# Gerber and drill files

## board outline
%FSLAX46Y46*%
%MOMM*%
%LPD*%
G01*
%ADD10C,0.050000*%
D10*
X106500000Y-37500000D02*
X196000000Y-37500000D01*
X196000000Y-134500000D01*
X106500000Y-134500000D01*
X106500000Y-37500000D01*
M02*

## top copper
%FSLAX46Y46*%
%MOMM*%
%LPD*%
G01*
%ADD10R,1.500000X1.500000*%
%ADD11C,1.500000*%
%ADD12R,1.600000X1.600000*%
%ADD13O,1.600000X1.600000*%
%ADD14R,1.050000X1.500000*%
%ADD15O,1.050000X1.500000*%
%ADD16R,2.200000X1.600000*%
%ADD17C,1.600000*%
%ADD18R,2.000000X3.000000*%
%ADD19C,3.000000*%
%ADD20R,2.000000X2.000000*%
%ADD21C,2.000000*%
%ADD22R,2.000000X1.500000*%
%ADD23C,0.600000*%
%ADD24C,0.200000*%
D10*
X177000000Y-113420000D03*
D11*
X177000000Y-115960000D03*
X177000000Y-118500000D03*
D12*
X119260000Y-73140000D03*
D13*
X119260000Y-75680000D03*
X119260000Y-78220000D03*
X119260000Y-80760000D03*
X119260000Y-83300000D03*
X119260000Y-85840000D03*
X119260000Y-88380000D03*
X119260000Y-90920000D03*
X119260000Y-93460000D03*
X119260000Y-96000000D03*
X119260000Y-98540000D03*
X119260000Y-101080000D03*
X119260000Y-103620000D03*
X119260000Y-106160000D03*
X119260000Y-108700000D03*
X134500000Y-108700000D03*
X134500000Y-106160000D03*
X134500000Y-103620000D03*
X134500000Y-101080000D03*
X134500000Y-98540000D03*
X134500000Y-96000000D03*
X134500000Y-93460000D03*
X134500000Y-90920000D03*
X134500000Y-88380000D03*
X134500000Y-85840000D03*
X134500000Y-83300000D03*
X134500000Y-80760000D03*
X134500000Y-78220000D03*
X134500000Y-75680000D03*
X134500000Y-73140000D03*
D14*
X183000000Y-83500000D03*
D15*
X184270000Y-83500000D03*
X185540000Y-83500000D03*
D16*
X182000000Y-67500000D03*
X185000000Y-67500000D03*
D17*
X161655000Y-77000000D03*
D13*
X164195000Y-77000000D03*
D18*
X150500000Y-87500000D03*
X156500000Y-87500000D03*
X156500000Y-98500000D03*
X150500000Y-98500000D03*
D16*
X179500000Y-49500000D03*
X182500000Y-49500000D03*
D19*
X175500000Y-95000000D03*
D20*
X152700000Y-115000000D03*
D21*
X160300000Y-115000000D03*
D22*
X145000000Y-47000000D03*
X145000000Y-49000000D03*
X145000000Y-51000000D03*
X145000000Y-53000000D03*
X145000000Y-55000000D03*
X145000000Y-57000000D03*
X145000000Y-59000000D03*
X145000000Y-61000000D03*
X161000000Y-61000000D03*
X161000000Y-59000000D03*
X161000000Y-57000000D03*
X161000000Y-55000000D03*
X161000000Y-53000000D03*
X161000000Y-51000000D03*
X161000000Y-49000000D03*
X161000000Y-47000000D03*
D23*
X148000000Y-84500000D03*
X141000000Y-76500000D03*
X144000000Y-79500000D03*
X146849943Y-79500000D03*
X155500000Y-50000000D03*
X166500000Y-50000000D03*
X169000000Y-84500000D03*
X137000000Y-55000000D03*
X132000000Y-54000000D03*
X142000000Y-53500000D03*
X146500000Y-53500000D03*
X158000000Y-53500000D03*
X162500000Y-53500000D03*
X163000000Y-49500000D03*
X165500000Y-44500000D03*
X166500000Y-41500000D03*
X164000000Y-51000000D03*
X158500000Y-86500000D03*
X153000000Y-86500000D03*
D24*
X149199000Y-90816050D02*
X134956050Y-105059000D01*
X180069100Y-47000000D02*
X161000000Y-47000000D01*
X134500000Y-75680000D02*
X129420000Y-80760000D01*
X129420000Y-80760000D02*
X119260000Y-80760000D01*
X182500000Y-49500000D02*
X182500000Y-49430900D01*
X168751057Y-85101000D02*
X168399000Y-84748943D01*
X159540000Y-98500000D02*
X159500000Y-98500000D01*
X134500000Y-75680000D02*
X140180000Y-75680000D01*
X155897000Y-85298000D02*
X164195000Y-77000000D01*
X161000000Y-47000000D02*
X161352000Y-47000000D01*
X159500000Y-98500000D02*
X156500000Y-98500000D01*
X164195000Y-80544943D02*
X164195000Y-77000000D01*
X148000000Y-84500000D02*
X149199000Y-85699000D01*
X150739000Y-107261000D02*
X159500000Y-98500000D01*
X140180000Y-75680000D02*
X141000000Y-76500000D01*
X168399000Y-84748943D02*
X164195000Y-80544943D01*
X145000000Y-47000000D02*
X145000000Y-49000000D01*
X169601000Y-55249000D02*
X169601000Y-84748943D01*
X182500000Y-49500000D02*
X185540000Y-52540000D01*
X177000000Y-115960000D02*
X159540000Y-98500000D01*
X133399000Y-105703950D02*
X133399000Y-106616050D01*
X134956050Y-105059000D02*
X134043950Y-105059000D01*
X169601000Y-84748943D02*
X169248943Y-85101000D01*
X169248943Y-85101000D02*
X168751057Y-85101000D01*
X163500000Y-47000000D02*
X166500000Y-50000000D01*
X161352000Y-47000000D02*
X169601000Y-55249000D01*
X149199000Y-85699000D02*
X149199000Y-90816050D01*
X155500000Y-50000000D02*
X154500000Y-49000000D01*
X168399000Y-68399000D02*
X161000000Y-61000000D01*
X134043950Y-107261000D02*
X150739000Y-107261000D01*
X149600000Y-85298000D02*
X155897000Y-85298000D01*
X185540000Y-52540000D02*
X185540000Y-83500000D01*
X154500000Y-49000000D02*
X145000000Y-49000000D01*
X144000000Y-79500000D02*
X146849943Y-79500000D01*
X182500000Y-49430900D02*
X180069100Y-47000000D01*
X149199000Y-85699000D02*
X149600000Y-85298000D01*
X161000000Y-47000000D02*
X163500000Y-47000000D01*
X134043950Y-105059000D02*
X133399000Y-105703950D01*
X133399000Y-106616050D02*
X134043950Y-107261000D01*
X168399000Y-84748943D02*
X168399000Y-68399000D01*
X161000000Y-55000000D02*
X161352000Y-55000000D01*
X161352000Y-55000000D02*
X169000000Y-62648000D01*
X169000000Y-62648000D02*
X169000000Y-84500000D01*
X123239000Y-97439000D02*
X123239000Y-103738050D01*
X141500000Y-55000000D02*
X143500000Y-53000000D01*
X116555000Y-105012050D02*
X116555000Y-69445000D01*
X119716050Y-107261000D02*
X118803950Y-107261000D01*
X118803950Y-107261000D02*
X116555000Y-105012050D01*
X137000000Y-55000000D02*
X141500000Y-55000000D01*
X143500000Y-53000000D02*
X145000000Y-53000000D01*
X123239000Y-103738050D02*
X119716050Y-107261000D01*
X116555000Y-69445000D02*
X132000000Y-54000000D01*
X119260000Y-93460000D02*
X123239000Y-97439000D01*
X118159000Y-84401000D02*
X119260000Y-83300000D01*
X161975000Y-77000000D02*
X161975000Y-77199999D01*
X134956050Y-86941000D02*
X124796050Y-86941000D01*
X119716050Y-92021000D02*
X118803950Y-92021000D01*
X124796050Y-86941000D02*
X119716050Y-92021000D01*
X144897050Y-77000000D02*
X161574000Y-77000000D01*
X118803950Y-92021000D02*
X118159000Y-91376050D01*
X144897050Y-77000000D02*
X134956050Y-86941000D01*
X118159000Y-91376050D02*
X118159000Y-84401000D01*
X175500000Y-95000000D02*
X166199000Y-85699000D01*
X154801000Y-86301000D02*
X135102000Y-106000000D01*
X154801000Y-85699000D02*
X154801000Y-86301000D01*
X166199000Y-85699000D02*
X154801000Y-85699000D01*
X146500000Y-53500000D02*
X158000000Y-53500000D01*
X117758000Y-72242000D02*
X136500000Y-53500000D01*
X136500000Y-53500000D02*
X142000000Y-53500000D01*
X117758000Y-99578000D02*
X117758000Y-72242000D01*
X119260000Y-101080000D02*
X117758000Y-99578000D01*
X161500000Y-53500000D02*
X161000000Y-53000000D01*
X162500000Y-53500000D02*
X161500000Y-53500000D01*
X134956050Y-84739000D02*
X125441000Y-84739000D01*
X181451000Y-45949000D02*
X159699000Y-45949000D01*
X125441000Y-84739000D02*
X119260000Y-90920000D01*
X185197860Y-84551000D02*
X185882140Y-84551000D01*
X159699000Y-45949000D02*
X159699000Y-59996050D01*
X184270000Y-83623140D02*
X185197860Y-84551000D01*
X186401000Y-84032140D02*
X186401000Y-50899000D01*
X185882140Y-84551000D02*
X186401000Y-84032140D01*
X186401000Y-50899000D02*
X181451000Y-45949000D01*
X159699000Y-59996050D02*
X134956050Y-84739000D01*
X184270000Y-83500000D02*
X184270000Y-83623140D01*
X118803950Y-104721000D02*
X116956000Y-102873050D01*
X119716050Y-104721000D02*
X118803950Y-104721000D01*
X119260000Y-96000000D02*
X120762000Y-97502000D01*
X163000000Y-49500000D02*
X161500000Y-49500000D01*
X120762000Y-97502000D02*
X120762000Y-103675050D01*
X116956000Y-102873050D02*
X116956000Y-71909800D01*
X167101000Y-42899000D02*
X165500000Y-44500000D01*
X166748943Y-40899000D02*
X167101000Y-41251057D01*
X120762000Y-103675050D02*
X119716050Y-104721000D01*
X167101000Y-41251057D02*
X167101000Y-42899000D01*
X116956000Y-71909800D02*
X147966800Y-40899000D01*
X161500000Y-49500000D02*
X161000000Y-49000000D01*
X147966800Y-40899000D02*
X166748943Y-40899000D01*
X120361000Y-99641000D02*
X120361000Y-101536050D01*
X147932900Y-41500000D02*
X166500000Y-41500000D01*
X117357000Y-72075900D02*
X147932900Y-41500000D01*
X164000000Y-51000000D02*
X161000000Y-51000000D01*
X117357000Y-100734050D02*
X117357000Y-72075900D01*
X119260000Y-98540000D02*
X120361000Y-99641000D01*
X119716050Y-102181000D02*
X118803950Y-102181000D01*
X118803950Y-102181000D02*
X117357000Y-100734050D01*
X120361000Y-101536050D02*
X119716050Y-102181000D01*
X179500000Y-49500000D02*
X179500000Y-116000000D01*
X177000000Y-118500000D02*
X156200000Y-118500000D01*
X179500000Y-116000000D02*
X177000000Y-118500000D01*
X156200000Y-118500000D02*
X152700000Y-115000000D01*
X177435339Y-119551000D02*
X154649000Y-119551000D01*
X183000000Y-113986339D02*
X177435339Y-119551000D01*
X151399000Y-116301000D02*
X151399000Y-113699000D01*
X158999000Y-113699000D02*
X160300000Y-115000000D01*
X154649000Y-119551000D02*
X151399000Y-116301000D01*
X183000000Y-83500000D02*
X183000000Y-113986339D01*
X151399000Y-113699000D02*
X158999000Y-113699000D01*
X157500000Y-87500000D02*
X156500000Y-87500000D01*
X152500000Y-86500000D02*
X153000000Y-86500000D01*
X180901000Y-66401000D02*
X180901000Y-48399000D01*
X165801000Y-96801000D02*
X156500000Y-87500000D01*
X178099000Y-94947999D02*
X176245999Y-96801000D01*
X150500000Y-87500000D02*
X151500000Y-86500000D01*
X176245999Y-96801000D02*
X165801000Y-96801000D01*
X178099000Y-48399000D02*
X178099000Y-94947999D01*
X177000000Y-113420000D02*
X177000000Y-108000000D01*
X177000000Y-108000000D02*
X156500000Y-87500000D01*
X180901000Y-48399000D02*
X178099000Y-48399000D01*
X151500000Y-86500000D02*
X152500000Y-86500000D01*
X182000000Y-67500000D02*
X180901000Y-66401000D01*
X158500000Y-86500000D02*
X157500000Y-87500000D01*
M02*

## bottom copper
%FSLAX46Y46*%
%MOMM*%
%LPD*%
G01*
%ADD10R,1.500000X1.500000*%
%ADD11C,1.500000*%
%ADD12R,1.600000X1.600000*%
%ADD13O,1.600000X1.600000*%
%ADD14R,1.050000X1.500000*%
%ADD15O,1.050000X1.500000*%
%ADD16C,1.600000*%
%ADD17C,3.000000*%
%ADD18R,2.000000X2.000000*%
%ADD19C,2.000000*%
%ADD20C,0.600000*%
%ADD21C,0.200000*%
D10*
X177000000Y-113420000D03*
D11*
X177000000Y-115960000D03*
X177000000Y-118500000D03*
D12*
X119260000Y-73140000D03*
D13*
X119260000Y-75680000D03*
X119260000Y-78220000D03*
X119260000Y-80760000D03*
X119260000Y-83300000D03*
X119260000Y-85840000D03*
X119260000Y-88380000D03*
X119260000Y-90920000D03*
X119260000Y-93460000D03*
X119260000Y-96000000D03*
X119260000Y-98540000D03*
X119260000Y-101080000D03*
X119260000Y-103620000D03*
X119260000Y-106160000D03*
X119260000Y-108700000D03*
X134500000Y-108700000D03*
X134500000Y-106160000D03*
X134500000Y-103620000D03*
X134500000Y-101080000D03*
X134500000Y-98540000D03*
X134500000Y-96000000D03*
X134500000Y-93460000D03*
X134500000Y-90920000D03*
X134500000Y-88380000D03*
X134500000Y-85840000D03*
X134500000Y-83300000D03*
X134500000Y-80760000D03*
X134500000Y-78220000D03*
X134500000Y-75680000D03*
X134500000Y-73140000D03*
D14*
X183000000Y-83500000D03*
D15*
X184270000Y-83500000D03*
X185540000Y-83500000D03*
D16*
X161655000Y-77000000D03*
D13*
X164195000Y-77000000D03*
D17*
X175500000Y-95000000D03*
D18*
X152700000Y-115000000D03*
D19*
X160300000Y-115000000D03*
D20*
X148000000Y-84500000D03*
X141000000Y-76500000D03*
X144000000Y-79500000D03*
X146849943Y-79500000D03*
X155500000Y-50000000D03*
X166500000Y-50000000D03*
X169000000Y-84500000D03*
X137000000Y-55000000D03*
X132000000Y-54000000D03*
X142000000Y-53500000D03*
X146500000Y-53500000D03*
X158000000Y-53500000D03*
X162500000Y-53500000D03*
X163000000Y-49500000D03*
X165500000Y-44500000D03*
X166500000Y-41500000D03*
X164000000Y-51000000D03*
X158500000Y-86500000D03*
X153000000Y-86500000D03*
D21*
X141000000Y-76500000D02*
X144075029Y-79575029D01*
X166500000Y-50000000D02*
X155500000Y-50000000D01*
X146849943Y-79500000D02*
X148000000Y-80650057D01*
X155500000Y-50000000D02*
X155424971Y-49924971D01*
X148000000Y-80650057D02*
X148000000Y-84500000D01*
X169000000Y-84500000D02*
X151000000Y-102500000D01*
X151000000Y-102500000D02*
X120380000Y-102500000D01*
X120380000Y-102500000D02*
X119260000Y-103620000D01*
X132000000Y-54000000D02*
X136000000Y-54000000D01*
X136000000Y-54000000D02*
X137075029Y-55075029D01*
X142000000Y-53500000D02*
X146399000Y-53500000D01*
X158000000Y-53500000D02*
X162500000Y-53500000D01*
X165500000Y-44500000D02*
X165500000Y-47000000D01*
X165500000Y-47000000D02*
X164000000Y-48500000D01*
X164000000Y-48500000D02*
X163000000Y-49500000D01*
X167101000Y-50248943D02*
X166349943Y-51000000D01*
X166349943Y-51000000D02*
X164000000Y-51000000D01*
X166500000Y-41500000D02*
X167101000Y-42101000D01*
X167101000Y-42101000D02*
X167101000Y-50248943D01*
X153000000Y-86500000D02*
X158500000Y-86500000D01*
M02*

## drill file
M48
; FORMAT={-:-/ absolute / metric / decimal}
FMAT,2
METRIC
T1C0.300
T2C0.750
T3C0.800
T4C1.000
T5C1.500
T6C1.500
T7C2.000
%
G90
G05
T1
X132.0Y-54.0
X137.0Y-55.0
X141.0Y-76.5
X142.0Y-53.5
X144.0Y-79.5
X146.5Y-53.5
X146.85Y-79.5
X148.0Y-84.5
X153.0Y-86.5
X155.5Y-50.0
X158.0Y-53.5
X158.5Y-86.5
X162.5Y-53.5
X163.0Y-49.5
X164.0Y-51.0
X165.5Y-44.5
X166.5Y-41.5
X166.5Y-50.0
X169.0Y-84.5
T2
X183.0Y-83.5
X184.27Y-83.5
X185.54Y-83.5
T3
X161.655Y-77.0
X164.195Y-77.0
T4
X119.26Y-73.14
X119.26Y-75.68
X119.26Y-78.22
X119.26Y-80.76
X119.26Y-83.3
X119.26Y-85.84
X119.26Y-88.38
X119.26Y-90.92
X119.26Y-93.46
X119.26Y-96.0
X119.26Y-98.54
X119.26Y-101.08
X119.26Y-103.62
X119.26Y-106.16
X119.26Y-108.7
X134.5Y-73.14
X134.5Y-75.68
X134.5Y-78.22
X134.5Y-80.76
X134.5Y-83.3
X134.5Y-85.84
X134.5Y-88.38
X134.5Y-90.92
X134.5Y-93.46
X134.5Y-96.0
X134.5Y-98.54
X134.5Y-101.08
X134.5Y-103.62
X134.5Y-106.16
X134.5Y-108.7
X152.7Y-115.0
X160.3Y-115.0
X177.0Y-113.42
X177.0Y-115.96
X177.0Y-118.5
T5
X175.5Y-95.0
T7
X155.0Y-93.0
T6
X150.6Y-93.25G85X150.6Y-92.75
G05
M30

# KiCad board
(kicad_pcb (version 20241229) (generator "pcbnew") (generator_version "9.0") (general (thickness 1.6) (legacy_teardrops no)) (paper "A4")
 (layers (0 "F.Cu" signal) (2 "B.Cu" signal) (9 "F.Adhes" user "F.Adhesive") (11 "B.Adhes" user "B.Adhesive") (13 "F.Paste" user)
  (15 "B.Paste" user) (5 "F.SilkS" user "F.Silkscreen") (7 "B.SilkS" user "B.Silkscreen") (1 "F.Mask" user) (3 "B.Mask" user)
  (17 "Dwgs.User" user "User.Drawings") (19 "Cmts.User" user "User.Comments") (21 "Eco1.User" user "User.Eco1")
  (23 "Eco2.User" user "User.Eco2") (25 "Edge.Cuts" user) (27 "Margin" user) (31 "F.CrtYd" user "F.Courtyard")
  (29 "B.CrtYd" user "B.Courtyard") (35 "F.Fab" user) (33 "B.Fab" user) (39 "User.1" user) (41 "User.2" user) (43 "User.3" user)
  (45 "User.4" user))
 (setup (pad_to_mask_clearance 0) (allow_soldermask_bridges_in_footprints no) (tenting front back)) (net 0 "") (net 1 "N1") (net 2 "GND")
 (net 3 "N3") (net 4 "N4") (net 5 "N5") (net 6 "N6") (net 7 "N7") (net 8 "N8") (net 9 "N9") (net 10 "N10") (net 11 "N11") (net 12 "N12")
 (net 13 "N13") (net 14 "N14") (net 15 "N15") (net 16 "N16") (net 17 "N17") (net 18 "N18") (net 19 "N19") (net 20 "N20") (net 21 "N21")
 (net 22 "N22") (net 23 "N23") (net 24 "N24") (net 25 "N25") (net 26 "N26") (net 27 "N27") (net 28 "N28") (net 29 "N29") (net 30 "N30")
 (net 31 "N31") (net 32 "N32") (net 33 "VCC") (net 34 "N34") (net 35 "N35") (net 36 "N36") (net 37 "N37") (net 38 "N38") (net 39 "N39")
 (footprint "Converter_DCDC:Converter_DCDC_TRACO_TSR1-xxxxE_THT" (layer "F.Cu") (at 177 113.42)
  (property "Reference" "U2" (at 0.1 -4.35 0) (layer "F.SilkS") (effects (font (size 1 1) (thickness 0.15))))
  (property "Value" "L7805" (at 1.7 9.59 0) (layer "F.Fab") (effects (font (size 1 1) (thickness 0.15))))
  (pad "1" thru_hole rect (at 0 0) (size 1.5 1.5) (drill 1) (layers "*.Cu" "*.Mask") (remove_unused_layers no) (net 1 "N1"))
  (pad "2" thru_hole circle (at 0 2.54) (size 1.5 1.5) (drill 1) (layers "*.Cu" "*.Mask") (remove_unused_layers no) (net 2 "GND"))
  (pad "3" thru_hole circle (at 0 5.08) (size 1.5 1.5) (drill 1) (layers "*.Cu" "*.Mask") (remove_unused_layers no) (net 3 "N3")))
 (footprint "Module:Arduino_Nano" (layer "F.Cu") (at 119.26 73.14)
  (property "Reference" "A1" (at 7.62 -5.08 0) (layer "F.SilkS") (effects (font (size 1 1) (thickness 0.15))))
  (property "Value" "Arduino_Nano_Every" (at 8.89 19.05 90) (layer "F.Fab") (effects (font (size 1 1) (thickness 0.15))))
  (pad "1" thru_hole rect (at 0 0) (size 1.6 1.6) (drill 1) (layers "*.Cu" "*.Mask") (remove_unused_layers no) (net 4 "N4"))
  (pad "2" thru_hole oval (at 0 2.54) (size 1.6 1.6) (drill 1) (layers "*.Cu" "*.Mask") (remove_unused_layers no) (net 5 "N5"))
  (pad "3" thru_hole oval (at 0 5.08) (size 1.6 1.6) (drill 1) (layers "*.Cu" "*.Mask") (remove_unused_layers no) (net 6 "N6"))
  (pad "4" thru_hole oval (at 0 7.62) (size 1.6 1.6) (drill 1) (layers "*.Cu" "*.Mask") (remove_unused_layers no) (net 2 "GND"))
  (pad "5" thru_hole oval (at 0 10.16) (size 1.6 1.6) (drill 1) (layers "*.Cu" "*.Mask") (remove_unused_layers no) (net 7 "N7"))
  (pad "6" thru_hole oval (at 0 12.7) (size 1.6 1.6) (drill 1) (layers "*.Cu" "*.Mask") (remove_unused_layers no) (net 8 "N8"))
  (pad "7" thru_hole oval (at 0 15.24) (size 1.6 1.6) (drill 1) (layers "*.Cu" "*.Mask") (remove_unused_layers no) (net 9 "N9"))
  (pad "8" thru_hole oval (at 0 17.78) (size 1.6 1.6) (drill 1) (layers "*.Cu" "*.Mask") (remove_unused_layers no) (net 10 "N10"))
  (pad "9" thru_hole oval (at 0 20.32) (size 1.6 1.6) (drill 1) (layers "*.Cu" "*.Mask") (remove_unused_layers no) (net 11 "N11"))
  (pad "10" thru_hole oval (at 0 22.86) (size 1.6 1.6) (drill 1) (layers "*.Cu" "*.Mask") (remove_unused_layers no) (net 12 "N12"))
  (pad "11" thru_hole oval (at 0 25.4) (size 1.6 1.6) (drill 1) (layers "*.Cu" "*.Mask") (remove_unused_layers no) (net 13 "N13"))
  (pad "12" thru_hole oval (at 0 27.94) (size 1.6 1.6) (drill 1) (layers "*.Cu" "*.Mask") (remove_unused_layers no) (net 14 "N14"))
  (pad "13" thru_hole oval (at 0 30.48) (size 1.6 1.6) (drill 1) (layers "*.Cu" "*.Mask") (remove_unused_layers no) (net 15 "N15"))
  (pad "14" thru_hole oval (at 0 33.02) (size 1.6 1.6) (drill 1) (layers "*.Cu" "*.Mask") (remove_unused_layers no) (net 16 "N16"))
  (pad "15" thru_hole oval (at 0 35.56) (size 1.6 1.6) (drill 1) (layers "*.Cu" "*.Mask") (remove_unused_layers no) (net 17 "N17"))
  (pad "16" thru_hole oval (at 15.24 35.56) (size 1.6 1.6) (drill 1) (layers "*.Cu" "*.Mask") (remove_unused_layers no) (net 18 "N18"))
  (pad "17" thru_hole oval (at 15.24 33.02) (size 1.6 1.6) (drill 1) (layers "*.Cu" "*.Mask") (remove_unused_layers no) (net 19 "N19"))
  (pad "18" thru_hole oval (at 15.24 30.48) (size 1.6 1.6) (drill 1) (layers "*.Cu" "*.Mask") (remove_unused_layers no) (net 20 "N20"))
  (pad "19" thru_hole oval (at 15.24 27.94) (size 1.6 1.6) (drill 1) (layers "*.Cu" "*.Mask") (remove_unused_layers no) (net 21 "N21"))
  (pad "20" thru_hole oval (at 15.24 25.4) (size 1.6 1.6) (drill 1) (layers "*.Cu" "*.Mask") (remove_unused_layers no) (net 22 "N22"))
  (pad "21" thru_hole oval (at 15.24 22.86) (size 1.6 1.6) (drill 1) (layers "*.Cu" "*.Mask") (remove_unused_layers no) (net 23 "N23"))
  (pad "22" thru_hole oval (at 15.24 20.32) (size 1.6 1.6) (drill 1) (layers "*.Cu" "*.Mask") (remove_unused_layers no) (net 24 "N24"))
  (pad "23" thru_hole oval (at 15.24 17.78) (size 1.6 1.6) (drill 1) (layers "*.Cu" "*.Mask") (remove_unused_layers no) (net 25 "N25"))
  (pad "24" thru_hole oval (at 15.24 15.24) (size 1.6 1.6) (drill 1) (layers "*.Cu" "*.Mask") (remove_unused_layers no) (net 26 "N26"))
  (pad "25" thru_hole oval (at 15.24 12.7) (size 1.6 1.6) (drill 1) (layers "*.Cu" "*.Mask") (remove_unused_layers no) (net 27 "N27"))
  (pad "26" thru_hole oval (at 15.24 10.16) (size 1.6 1.6) (drill 1) (layers "*.Cu" "*.Mask") (remove_unused_layers no) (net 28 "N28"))
  (pad "27" thru_hole oval (at 15.24 7.62) (size 1.6 1.6) (drill 1) (layers "*.Cu" "*.Mask") (remove_unused_layers no) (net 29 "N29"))
  (pad "28" thru_hole oval (at 15.24 5.08) (size 1.6 1.6) (drill 1) (layers "*.Cu" "*.Mask") (remove_unused_layers no) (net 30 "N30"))
  (pad "29" thru_hole oval (at 15.24 2.54) (size 1.6 1.6) (drill 1) (layers "*.Cu" "*.Mask") (remove_unused_layers no) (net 2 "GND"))
  (pad "30" thru_hole oval (at 15.24 0) (size 1.6 1.6) (drill 1) (layers "*.Cu" "*.Mask") (remove_unused_layers no) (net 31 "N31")))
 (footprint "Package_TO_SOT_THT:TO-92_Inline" (layer "F.Cu") (at 183 83.5)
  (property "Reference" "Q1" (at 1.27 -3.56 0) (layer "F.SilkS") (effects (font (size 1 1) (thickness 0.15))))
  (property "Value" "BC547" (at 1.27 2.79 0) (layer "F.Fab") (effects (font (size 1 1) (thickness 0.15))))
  (pad "1" thru_hole rect (at 0 0) (size 1.05 1.5) (drill 0.75) (layers "*.Cu" "*.Mask") (remove_unused_layers no) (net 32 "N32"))
  (pad "2" thru_hole oval (at 1.27 0) (size 1.05 1.5) (drill 0.75) (layers "*.Cu" "*.Mask") (remove_unused_layers no) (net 10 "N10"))
  (pad "3" thru_hole oval (at 2.54 0) (size 1.05 1.5) (drill 0.75) (layers "*.Cu" "*.Mask") (remove_unused_layers no) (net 2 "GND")))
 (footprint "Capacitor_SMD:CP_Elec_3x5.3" (layer "F.Cu") (at 183.5 67.5)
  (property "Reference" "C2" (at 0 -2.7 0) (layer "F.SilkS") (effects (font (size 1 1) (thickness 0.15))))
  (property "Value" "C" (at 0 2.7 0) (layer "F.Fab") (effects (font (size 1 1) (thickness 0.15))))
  (pad "1" smd rect (at -1.5 0) (size 2.2 1.6) (layers "F.Cu" "F.Mask" "F.Paste") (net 1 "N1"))
  (pad "2" smd rect (at 1.5 0) (size 2.2 1.6) (layers "F.Cu" "F.Mask" "F.Paste") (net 2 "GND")))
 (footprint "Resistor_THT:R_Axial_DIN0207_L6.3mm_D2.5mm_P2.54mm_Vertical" (layer "F.Cu") (at 161.655 77)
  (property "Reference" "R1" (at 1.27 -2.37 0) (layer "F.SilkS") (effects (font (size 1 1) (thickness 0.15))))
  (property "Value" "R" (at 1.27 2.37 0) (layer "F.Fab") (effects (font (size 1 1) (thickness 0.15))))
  (pad "1" thru_hole circle (at 0 0) (size 1.6 1.6) (drill 0.8) (layers "*.Cu" "*.Mask") (remove_unused_layers no) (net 7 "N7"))
  (pad "2" thru_hole oval (at 2.54 0) (size 1.6 1.6) (drill 0.8) (layers "*.Cu" "*.Mask") (remove_unused_layers no) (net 2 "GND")))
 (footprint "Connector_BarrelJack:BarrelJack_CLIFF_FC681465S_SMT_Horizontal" (layer "F.Cu") (at 153.5 93)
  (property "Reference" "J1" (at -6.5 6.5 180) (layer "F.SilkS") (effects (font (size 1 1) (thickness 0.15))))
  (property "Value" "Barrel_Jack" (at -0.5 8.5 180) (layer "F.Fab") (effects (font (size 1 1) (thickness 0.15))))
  (pad "" np_thru_hole oval (at -2.9 0 90) (size 2 1.5) (drill oval 2 1.5) (layers "*.Cu" "*.Mask"))
  (pad "" np_thru_hole circle (at 1.5 0 90) (size 2 2) (drill 2) (layers "*.Cu" "*.Mask"))
  (pad "1" smd rect (at -3 -5.5 90) (size 3 2) (layers "F.Cu" "F.Mask" "F.Paste") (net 1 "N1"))
  (pad "1" smd rect (at 3 -5.5 90) (size 3 2) (layers "F.Cu" "F.Mask" "F.Paste") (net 1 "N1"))
  (pad "2" smd rect (at 3 5.5 90) (size 3 2) (layers "F.Cu" "F.Mask" "F.Paste") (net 2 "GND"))
  (pad "3" smd rect (at -3 5.5 90) (size 3 2) (layers "F.Cu" "F.Mask" "F.Paste")))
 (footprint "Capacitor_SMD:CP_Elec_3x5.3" (layer "F.Cu") (at 181 49.5)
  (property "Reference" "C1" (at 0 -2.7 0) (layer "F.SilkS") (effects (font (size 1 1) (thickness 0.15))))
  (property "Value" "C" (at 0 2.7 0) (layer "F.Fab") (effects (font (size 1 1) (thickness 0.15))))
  (pad "1" smd rect (at -1.5 0) (size 2.2 1.6) (layers "F.Cu" "F.Mask" "F.Paste") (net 3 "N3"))
  (pad "2" smd rect (at 1.5 0) (size 2.2 1.6) (layers "F.Cu" "F.Mask" "F.Paste") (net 2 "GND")))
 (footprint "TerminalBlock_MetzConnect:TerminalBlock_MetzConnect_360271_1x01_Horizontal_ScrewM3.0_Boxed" (layer "F.Cu") (at 175.5 95)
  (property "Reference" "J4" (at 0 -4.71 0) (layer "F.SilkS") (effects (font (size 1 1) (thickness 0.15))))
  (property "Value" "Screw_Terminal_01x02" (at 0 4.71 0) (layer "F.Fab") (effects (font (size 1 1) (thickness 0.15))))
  (pad "1" thru_hole circle (at 0 0) (size 3 3) (drill 1.5) (layers "*.Cu" "*.Mask") (remove_unused_layers no) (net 19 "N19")))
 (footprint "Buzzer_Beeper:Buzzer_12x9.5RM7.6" (layer "F.Cu") (at 152.7 115)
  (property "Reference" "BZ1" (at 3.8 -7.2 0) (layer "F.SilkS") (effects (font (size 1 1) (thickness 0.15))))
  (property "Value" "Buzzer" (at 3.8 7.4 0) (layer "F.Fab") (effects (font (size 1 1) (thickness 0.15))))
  (pad "1" thru_hole rect (at 0 0) (size 2 2) (drill 1) (layers "*.Cu" "*.Mask") (remove_unused_layers no) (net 3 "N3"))
  (pad "2" thru_hole circle (at 7.6 0) (size 2 2) (drill 1) (layers "*.Cu" "*.Mask") (remove_unused_layers no) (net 32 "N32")))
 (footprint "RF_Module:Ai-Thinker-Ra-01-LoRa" (layer "F.Cu") (at 153 54)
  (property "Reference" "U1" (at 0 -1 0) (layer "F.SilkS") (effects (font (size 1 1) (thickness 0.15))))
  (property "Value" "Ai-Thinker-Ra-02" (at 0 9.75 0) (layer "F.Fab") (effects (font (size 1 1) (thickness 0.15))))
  (pad "1" smd rect (at -8 -7) (size 2 1.5) (layers "F.Cu" "F.Mask" "F.Paste") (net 2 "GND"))
  (pad "2" smd rect (at -8 -5) (size 2 1.5) (layers "F.Cu" "F.Mask" "F.Paste") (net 2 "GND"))
  (pad "3" smd rect (at -8 -3) (size 2 1.5) (layers "F.Cu" "F.Mask" "F.Paste") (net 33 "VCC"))
  (pad "4" smd rect (at -8 -1) (size 2 1.5) (layers "F.Cu" "F.Mask" "F.Paste") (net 11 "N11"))
  (pad "5" smd rect (at -8 1) (size 2 1.5) (layers "F.Cu" "F.Mask" "F.Paste") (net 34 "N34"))
  (pad "6" smd rect (at -8 3) (size 2 1.5) (layers "F.Cu" "F.Mask" "F.Paste") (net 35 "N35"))
  (pad "7" smd rect (at -8 5) (size 2 1.5) (layers "F.Cu" "F.Mask" "F.Paste") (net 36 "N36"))
  (pad "8" smd rect (at -8 7) (size 2 1.5) (layers "F.Cu" "F.Mask" "F.Paste") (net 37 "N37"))
  (pad "9" smd rect (at 8 7) (size 2 1.5) (layers "F.Cu" "F.Mask" "F.Paste") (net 2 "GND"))
  (pad "10" smd rect (at 8 5) (size 2 1.5) (layers "F.Cu" "F.Mask" "F.Paste") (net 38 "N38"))
  (pad "11" smd rect (at 8 3) (size 2 1.5) (layers "F.Cu" "F.Mask" "F.Paste") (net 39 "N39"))
  (pad "12" smd rect (at 8 1) (size 2 1.5) (layers "F.Cu" "F.Mask" "F.Paste") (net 15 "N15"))
  (pad "13" smd rect (at 8 -1) (size 2 1.5) (layers "F.Cu" "F.Mask" "F.Paste") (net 14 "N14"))
  (pad "14" smd rect (at 8 -3) (size 2 1.5) (layers "F.Cu" "F.Mask" "F.Paste") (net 13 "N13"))
  (pad "15" smd rect (at 8 -5) (size 2 1.5) (layers "F.Cu" "F.Mask" "F.Paste") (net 12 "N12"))
  (pad "16" smd rect (at 8 -7) (size 2 1.5) (layers "F.Cu" "F.Mask" "F.Paste") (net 2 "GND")))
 (gr_rect (start 106.5 37.5) (end 196 134.5) (stroke (width 0.05) (type default)) (fill no) (layer "Edge.Cuts"))
 (segment (start 149.199 90.81605) (end 134.95605 105.059) (width 0.2) (layer "F.Cu") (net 2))
 (segment (start 180.0691 47) (end 161 47) (width 0.2) (layer "F.Cu") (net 2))
 (segment (start 134.5 75.68) (end 129.42 80.76) (width 0.2) (layer "F.Cu") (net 2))
 (segment (start 129.42 80.76) (end 119.26 80.76) (width 0.2) (layer "F.Cu") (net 2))
 (segment (start 182.5 49.5) (end 182.5 49.4309) (width 0.2) (layer "F.Cu") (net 2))
 (segment (start 168.751057 85.101) (end 168.399 84.748943) (width 0.2) (layer "F.Cu") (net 2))
 (segment (start 159.54 98.5) (end 159.5 98.5) (width 0.2) (layer "F.Cu") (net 2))
 (segment (start 134.5 75.68) (end 140.18 75.68) (width 0.2) (layer "F.Cu") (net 2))
 (segment (start 155.897 85.298) (end 164.195 77) (width 0.2) (layer "F.Cu") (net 2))
 (segment (start 161 47) (end 161.352 47) (width 0.2) (layer "F.Cu") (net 2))
 (segment (start 159.5 98.5) (end 156.5 98.5) (width 0.2) (layer "F.Cu") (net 2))
 (segment (start 164.195 80.544943) (end 164.195 77) (width 0.2) (layer "F.Cu") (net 2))
 (segment (start 148 84.5) (end 149.199 85.699) (width 0.2) (layer "F.Cu") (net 2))
 (segment (start 150.739 107.261) (end 159.5 98.5) (width 0.2) (layer "F.Cu") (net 2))
 (segment (start 140.18 75.68) (end 141 76.5) (width 0.2) (layer "F.Cu") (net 2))
 (segment (start 168.399 84.748943) (end 164.195 80.544943) (width 0.2) (layer "F.Cu") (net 2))
 (segment (start 145 47) (end 145 49) (width 0.2) (layer "F.Cu") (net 2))
 (segment (start 169.601 55.249) (end 169.601 84.748943) (width 0.2) (layer "F.Cu") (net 2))
 (segment (start 182.5 49.5) (end 185.54 52.54) (width 0.2) (layer "F.Cu") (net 2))
 (segment (start 177 115.96) (end 159.54 98.5) (width 0.2) (layer "F.Cu") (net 2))
 (segment (start 133.399 105.70395) (end 133.399 106.61605) (width 0.2) (layer "F.Cu") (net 2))
 (segment (start 134.95605 105.059) (end 134.04395 105.059) (width 0.2) (layer "F.Cu") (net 2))
 (segment (start 169.601 84.748943) (end 169.248943 85.101) (width 0.2) (layer "F.Cu") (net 2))
 (segment (start 169.248943 85.101) (end 168.751057 85.101) (width 0.2) (layer "F.Cu") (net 2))
 (segment (start 163.5 47) (end 166.5 50) (width 0.2) (layer "F.Cu") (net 2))
 (segment (start 161.352 47) (end 169.601 55.249) (width 0.2) (layer "F.Cu") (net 2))
 (segment (start 149.199 85.699) (end 149.199 90.81605) (width 0.2) (layer "F.Cu") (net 2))
 (segment (start 155.5 50) (end 154.5 49) (width 0.2) (layer "F.Cu") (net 2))
 (segment (start 168.399 68.399) (end 161 61) (width 0.2) (layer "F.Cu") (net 2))
 (segment (start 134.04395 107.261) (end 150.739 107.261) (width 0.2) (layer "F.Cu") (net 2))
 (segment (start 149.6 85.298) (end 155.897 85.298) (width 0.2) (layer "F.Cu") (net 2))
 (segment (start 185.54 52.54) (end 185.54 83.5) (width 0.2) (layer "F.Cu") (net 2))
 (segment (start 154.5 49) (end 145 49) (width 0.2) (layer "F.Cu") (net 2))
 (segment (start 144 79.5) (end 146.849943 79.5) (width 0.2) (layer "F.Cu") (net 2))
 (segment (start 182.5 49.4309) (end 180.0691 47) (width 0.2) (layer "F.Cu") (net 2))
 (segment (start 149.199 85.699) (end 149.6 85.298) (width 0.2) (layer "F.Cu") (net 2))
 (segment (start 161 47) (end 163.5 47) (width 0.2) (layer "F.Cu") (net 2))
 (segment (start 134.04395 105.059) (end 133.399 105.70395) (width 0.2) (layer "F.Cu") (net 2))
 (segment (start 133.399 106.61605) (end 134.04395 107.261) (width 0.2) (layer "F.Cu") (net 2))
 (segment (start 168.399 84.748943) (end 168.399 68.399) (width 0.2) (layer "F.Cu") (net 2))
 (via (at 148 84.5) (size 0.6) (drill 0.3) (layers "F.Cu" "B.Cu") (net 2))
 (via (at 141 76.5) (size 0.6) (drill 0.3) (layers "F.Cu" "B.Cu") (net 2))
 (via (at 144 79.5) (size 0.6) (drill 0.3) (layers "F.Cu" "B.Cu") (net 2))
 (via (at 146.849943 79.5) (size 0.6) (drill 0.3) (layers "F.Cu" "B.Cu") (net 2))
 (via (at 155.5 50) (size 0.6) (drill 0.3) (layers "F.Cu" "B.Cu") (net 2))
 (via (at 166.5 50) (size 0.6) (drill 0.3) (layers "F.Cu" "B.Cu") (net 2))
 (segment (start 141 76.5) (end 144.075029 79.575029) (width 0.2) (layer "B.Cu") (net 2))
 (segment (start 166.5 50) (end 155.5 50) (width 0.2) (layer "B.Cu") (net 2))
 (segment (start 146.849943 79.5) (end 148 80.650057) (width 0.2) (layer "B.Cu") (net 2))
 (segment (start 155.5 50) (end 155.424971 49.924971) (width 0.2) (layer "B.Cu") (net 2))
 (segment (start 148 80.650057) (end 148 84.5) (width 0.2) (layer "B.Cu") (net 2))
 (segment (start 161 55) (end 161.352 55) (width 0.2) (layer "F.Cu") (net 15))
 (segment (start 161.352 55) (end 169 62.648) (width 0.2) (layer "F.Cu") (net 15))
 (segment (start 169 62.648) (end 169 84.5) (width 0.2) (layer "F.Cu") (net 15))
 (via (at 169 84.5) (size 0.6) (drill 0.3) (layers "F.Cu" "B.Cu") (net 15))
 (segment (start 169 84.5) (end 151 102.5) (width 0.2) (layer "B.Cu") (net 15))
 (segment (start 151 102.5) (end 120.38 102.5) (width 0.2) (layer "B.Cu") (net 15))
 (segment (start 120.38 102.5) (end 119.26 103.62) (width 0.2) (layer "B.Cu") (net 15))
 (segment (start 123.239 97.439) (end 123.239 103.73805) (width 0.2) (layer "F.Cu") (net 11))
 (segment (start 141.5 55) (end 143.5 53) (width 0.2) (layer "F.Cu") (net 11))
 (segment (start 116.555 105.01205) (end 116.555 69.445) (width 0.2) (layer "F.Cu") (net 11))
 (segment (start 119.71605 107.261) (end 118.80395 107.261) (width 0.2) (layer "F.Cu") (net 11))
 (segment (start 118.80395 107.261) (end 116.555 105.01205) (width 0.2) (layer "F.Cu") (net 11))
 (segment (start 137 55) (end 141.5 55) (width 0.2) (layer "F.Cu") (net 11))
 (segment (start 143.5 53) (end 145 53) (width 0.2) (layer "F.Cu") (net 11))
 (segment (start 123.239 103.73805) (end 119.71605 107.261) (width 0.2) (layer "F.Cu") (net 11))
 (segment (start 116.555 69.445) (end 132 54) (width 0.2) (layer "F.Cu") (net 11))
 (segment (start 119.26 93.46) (end 123.239 97.439) (width 0.2) (layer "F.Cu") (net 11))
 (via (at 137 55) (size 0.6) (drill 0.3) (layers "F.Cu" "B.Cu") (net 11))
 (via (at 132 54) (size 0.6) (drill 0.3) (layers "F.Cu" "B.Cu") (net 11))
 (segment (start 132 54) (end 136 54) (width 0.2) (layer "B.Cu") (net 11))
 (segment (start 136 54) (end 137.075029 55.075029) (width 0.2) (layer "B.Cu") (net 11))
 (segment (start 118.159 84.401) (end 119.26 83.3) (width 0.2) (layer "F.Cu") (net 7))
 (segment (start 161.975 77) (end 161.975 77.199999) (width 0.2) (layer "F.Cu") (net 7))
 (segment (start 134.95605 86.941) (end 124.79605 86.941) (width 0.2) (layer "F.Cu") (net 7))
 (segment (start 119.71605 92.021) (end 118.80395 92.021) (width 0.2) (layer "F.Cu") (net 7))
 (segment (start 124.79605 86.941) (end 119.71605 92.021) (width 0.2) (layer "F.Cu") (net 7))
 (segment (start 144.89705 77) (end 161.574 77) (width 0.2) (layer "F.Cu") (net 7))
 (segment (start 118.80395 92.021) (end 118.159 91.37605) (width 0.2) (layer "F.Cu") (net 7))
 (segment (start 144.89705 77) (end 134.95605 86.941) (width 0.2) (layer "F.Cu") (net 7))
 (segment (start 118.159 91.37605) (end 118.159 84.401) (width 0.2) (layer "F.Cu") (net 7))
 (segment (start 175.5 95) (end 166.199 85.699) (width 0.2) (layer "F.Cu") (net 19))
 (segment (start 154.801 86.301) (end 135.102 106) (width 0.2) (layer "F.Cu") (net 19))
 (segment (start 154.801 85.699) (end 154.801 86.301) (width 0.2) (layer "F.Cu") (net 19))
 (segment (start 166.199 85.699) (end 154.801 85.699) (width 0.2) (layer "F.Cu") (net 19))
 (segment (start 146.5 53.5) (end 158 53.5) (width 0.2) (layer "F.Cu") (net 14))
 (segment (start 117.758 72.242) (end 136.5 53.5) (width 0.2) (layer "F.Cu") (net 14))
 (segment (start 136.5 53.5) (end 142 53.5) (width 0.2) (layer "F.Cu") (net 14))
 (segment (start 117.758 99.578) (end 117.758 72.242) (width 0.2) (layer "F.Cu") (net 14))
 (segment (start 119.26 101.08) (end 117.758 99.578) (width 0.2) (layer "F.Cu") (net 14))
 (segment (start 161.5 53.5) (end 161 53) (width 0.2) (layer "F.Cu") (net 14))
 (segment (start 162.5 53.5) (end 161.5 53.5) (width 0.2) (layer "F.Cu") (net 14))
 (via (at 142 53.5) (size 0.6) (drill 0.3) (layers "F.Cu" "B.Cu") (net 14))
 (via (at 146.5 53.5) (size 0.6) (drill 0.3) (layers "F.Cu" "B.Cu") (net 14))
 (via (at 158 53.5) (size 0.6) (drill 0.3) (layers "F.Cu" "B.Cu") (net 14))
 (via (at 162.5 53.5) (size 0.6) (drill 0.3) (layers "F.Cu" "B.Cu") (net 14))
 (segment (start 142 53.5) (end 146.399 53.5) (width 0.2) (layer "B.Cu") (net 14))
 (segment (start 158 53.5) (end 162.5 53.5) (width 0.2) (layer "B.Cu") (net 14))
 (segment (start 134.95605 84.739) (end 125.441 84.739) (width 0.2) (layer "F.Cu") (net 10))
 (segment (start 181.451 45.949) (end 159.699 45.949) (width 0.2) (layer "F.Cu") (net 10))
 (segment (start 125.441 84.739) (end 119.26 90.92) (width 0.2) (layer "F.Cu") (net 10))
 (segment (start 185.19786 84.551) (end 185.88214 84.551) (width 0.2) (layer "F.Cu") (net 10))
 (segment (start 159.699 45.949) (end 159.699 59.99605) (width 0.2) (layer "F.Cu") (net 10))
 (segment (start 184.27 83.62314) (end 185.19786 84.551) (width 0.2) (layer "F.Cu") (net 10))
 (segment (start 186.401 84.03214) (end 186.401 50.899) (width 0.2) (layer "F.Cu") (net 10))
 (segment (start 185.88214 84.551) (end 186.401 84.03214) (width 0.2) (layer "F.Cu") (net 10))
 (segment (start 186.401 50.899) (end 181.451 45.949) (width 0.2) (layer "F.Cu") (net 10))
 (segment (start 159.699 59.99605) (end 134.95605 84.739) (width 0.2) (layer "F.Cu") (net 10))
 (segment (start 184.27 83.5) (end 184.27 83.62314) (width 0.2) (layer "F.Cu") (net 10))
 (segment (start 118.80395 104.721) (end 116.956 102.87305) (width 0.2) (layer "F.Cu") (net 12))
 (segment (start 119.71605 104.721) (end 118.80395 104.721) (width 0.2) (layer "F.Cu") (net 12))
 (segment (start 119.26 96) (end 120.762 97.502) (width 0.2) (layer "F.Cu") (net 12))
 (segment (start 163 49.5) (end 161.5 49.5) (width 0.2) (layer "F.Cu") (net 12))
 (segment (start 120.762 97.502) (end 120.762 103.67505) (width 0.2) (layer "F.Cu") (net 12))
 (segment (start 116.956 102.87305) (end 116.956 71.9098) (width 0.2) (layer "F.Cu") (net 12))
 (segment (start 167.101 42.899) (end 165.5 44.5) (width 0.2) (layer "F.Cu") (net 12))
 (segment (start 166.748943 40.899) (end 167.101 41.251057) (width 0.2) (layer "F.Cu") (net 12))
 (segment (start 120.762 103.67505) (end 119.71605 104.721) (width 0.2) (layer "F.Cu") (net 12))
 (segment (start 167.101 41.251057) (end 167.101 42.899) (width 0.2) (layer "F.Cu") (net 12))
 (segment (start 116.956 71.9098) (end 147.9668 40.899) (width 0.2) (layer "F.Cu") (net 12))
 (segment (start 161.5 49.5) (end 161 49) (width 0.2) (layer "F.Cu") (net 12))
 (segment (start 147.9668 40.899) (end 166.748943 40.899) (width 0.2) (layer "F.Cu") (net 12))
 (via (at 163 49.5) (size 0.6) (drill 0.3) (layers "F.Cu" "B.Cu") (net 12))
 (via (at 165.5 44.5) (size 0.6) (drill 0.3) (layers "F.Cu" "B.Cu") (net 12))
 (segment (start 165.5 44.5) (end 165.5 47) (width 0.2) (layer "B.Cu") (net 12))
 (segment (start 165.5 47) (end 164 48.5) (width 0.2) (layer "B.Cu") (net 12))
 (segment (start 164 48.5) (end 163 49.5) (width 0.2) (layer "B.Cu") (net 12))
 (segment (start 120.361 99.641) (end 120.361 101.53605) (width 0.2) (layer "F.Cu") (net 13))
 (segment (start 147.9329 41.5) (end 166.5 41.5) (width 0.2) (layer "F.Cu") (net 13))
 (segment (start 117.357 72.0759) (end 147.9329 41.5) (width 0.2) (layer "F.Cu") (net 13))
 (segment (start 164 51) (end 161 51) (width 0.2) (layer "F.Cu") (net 13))
 (segment (start 117.357 100.73405) (end 117.357 72.0759) (width 0.2) (layer "F.Cu") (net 13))
 (segment (start 119.26 98.54) (end 120.361 99.641) (width 0.2) (layer "F.Cu") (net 13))
 (segment (start 119.71605 102.181) (end 118.80395 102.181) (width 0.2) (layer "F.Cu") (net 13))
 (segment (start 118.80395 102.181) (end 117.357 100.73405) (width 0.2) (layer "F.Cu") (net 13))
 (segment (start 120.361 101.53605) (end 119.71605 102.181) (width 0.2) (layer "F.Cu") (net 13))
 (via (at 166.5 41.5) (size 0.6) (drill 0.3) (layers "F.Cu" "B.Cu") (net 13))
 (via (at 164 51) (size 0.6) (drill 0.3) (layers "F.Cu" "B.Cu") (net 13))
 (segment (start 167.101 50.248943) (end 166.349943 51) (width 0.2) (layer "B.Cu") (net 13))
 (segment (start 166.349943 51) (end 164 51) (width 0.2) (layer "B.Cu") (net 13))
 (segment (start 166.5 41.5) (end 167.101 42.101) (width 0.2) (layer "B.Cu") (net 13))
 (segment (start 167.101 42.101) (end 167.101 50.248943) (width 0.2) (layer "B.Cu") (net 13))
 (segment (start 179.5 49.5) (end 179.5 116) (width 0.2) (layer "F.Cu") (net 3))
 (segment (start 177 118.5) (end 156.2 118.5) (width 0.2) (layer "F.Cu") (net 3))
 (segment (start 179.5 116) (end 177 118.5) (width 0.2) (layer "F.Cu") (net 3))
 (segment (start 156.2 118.5) (end 152.7 115) (width 0.2) (layer "F.Cu") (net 3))
 (segment (start 177.435339 119.551) (end 154.649 119.551) (width 0.2) (layer "F.Cu") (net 32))
 (segment (start 183 113.986339) (end 177.435339 119.551) (width 0.2) (layer "F.Cu") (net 32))
 (segment (start 151.399 116.301) (end 151.399 113.699) (width 0.2) (layer "F.Cu") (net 32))
 (segment (start 158.999 113.699) (end 160.3 115) (width 0.2) (layer "F.Cu") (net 32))
 (segment (start 154.649 119.551) (end 151.399 116.301) (width 0.2) (layer "F.Cu") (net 32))
 (segment (start 183 83.5) (end 183 113.986339) (width 0.2) (layer "F.Cu") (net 32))
 (segment (start 151.399 113.699) (end 158.999 113.699) (width 0.2) (layer "F.Cu") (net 32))
 (segment (start 157.5 87.5) (end 156.5 87.5) (width 0.2) (layer "F.Cu") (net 1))
 (segment (start 152.5 86.5) (end 153 86.5) (width 0.2) (layer "F.Cu") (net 1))
 (segment (start 180.901 66.401) (end 180.901 48.399) (width 0.2) (layer "F.Cu") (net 1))
 (segment (start 165.801 96.801) (end 156.5 87.5) (width 0.2) (layer "F.Cu") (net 1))
 (segment (start 178.099 94.947999) (end 176.245999 96.801) (width 0.2) (layer "F.Cu") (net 1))
 (segment (start 150.5 87.5) (end 151.5 86.5) (width 0.2) (layer "F.Cu") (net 1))
 (segment (start 176.245999 96.801) (end 165.801 96.801) (width 0.2) (layer "F.Cu") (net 1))
 (segment (start 178.099 48.399) (end 178.099 94.947999) (width 0.2) (layer "F.Cu") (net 1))
 (segment (start 177 113.42) (end 177 108) (width 0.2) (layer "F.Cu") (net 1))
 (segment (start 177 108) (end 156.5 87.5) (width 0.2) (layer "F.Cu") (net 1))
 (segment (start 180.901 48.399) (end 178.099 48.399) (width 0.2) (layer "F.Cu") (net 1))
 (segment (start 151.5 86.5) (end 152.5 86.5) (width 0.2) (layer "F.Cu") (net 1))
 (segment (start 182 67.5) (end 180.901 66.401) (width 0.2) (layer "F.Cu") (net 1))
 (segment (start 158.5 86.5) (end 157.5 87.5) (width 0.2) (layer "F.Cu") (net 1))
 (via (at 158.5 86.5) (size 0.6) (drill 0.3) (layers "F.Cu" "B.Cu") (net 1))
 (via (at 153 86.5) (size 0.6) (drill 0.3) (layers "F.Cu" "B.Cu") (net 1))
 (segment (start 153 86.5) (end 158.5 86.5) (width 0.2) (layer "B.Cu") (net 1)))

